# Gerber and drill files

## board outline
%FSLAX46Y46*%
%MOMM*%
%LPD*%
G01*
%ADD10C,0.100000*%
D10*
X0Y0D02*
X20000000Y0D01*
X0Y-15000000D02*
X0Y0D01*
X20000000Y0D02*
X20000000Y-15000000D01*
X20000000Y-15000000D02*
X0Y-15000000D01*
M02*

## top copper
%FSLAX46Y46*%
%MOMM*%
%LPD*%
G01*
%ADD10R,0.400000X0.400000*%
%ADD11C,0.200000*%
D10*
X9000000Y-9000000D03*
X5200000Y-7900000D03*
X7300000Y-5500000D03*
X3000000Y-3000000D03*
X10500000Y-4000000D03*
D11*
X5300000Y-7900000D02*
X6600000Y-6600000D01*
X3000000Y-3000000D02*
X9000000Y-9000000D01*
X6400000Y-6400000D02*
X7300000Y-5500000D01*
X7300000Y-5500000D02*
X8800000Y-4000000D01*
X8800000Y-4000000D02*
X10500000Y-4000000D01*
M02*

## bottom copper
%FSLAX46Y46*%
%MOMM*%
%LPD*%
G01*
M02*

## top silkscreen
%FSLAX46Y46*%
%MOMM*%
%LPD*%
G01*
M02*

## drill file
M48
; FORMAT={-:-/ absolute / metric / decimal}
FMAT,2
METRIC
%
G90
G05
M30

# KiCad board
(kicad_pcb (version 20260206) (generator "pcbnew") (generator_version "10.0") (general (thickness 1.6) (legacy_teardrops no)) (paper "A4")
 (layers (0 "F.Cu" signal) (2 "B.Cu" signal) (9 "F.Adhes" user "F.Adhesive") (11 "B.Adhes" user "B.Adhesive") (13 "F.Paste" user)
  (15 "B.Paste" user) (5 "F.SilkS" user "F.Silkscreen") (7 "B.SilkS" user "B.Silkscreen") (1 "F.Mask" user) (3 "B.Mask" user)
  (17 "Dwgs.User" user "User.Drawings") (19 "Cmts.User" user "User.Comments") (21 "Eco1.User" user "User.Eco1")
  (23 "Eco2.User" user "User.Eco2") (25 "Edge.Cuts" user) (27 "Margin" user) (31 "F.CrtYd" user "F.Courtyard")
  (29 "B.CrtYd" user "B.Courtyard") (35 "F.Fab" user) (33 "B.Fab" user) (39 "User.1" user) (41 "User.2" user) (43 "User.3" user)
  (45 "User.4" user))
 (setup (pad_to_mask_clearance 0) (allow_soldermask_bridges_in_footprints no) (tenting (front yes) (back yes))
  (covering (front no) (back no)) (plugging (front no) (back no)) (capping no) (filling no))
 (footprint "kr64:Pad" (layer "F.Cu") (at 9 9)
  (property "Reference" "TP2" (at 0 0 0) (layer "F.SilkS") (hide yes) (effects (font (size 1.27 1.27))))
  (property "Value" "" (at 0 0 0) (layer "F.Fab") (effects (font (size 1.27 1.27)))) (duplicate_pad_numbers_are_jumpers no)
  (pad "1" smd rect (at 0 0) (size 0.4 0.4) (layers "F.Cu" "F.Mask" "F.Paste") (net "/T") (thermal_bridge_angle 45)))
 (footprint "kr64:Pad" (layer "F.Cu") (at 5.2 7.9)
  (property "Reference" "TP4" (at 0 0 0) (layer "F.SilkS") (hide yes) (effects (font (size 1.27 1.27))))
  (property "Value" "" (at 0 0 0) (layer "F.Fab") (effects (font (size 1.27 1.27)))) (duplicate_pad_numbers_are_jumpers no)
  (pad "1" smd rect (at 0 0) (size 0.4 0.4) (layers "F.Cu" "F.Mask" "F.Paste") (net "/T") (thermal_bridge_angle 45)))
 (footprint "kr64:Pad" (layer "F.Cu") (at 7.3 5.5)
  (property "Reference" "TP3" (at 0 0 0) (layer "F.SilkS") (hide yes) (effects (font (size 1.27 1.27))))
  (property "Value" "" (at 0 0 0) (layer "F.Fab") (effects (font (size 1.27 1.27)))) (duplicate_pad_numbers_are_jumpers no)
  (pad "1" smd rect (at 0 0) (size 0.4 0.4) (layers "F.Cu" "F.Mask" "F.Paste") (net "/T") (thermal_bridge_angle 45)))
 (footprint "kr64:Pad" (layer "F.Cu") (at 3 3)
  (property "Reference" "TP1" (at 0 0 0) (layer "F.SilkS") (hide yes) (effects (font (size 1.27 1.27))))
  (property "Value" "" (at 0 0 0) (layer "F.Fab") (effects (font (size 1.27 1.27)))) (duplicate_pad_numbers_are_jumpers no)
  (pad "1" smd rect (at 0 0) (size 0.4 0.4) (layers "F.Cu" "F.Mask" "F.Paste") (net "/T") (thermal_bridge_angle 45)))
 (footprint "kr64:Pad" (layer "F.Cu") (at 10.5 4)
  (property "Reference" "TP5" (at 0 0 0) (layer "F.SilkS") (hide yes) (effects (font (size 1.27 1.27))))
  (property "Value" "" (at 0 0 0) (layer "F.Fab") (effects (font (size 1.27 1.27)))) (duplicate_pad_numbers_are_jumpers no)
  (pad "1" smd rect (at 0 0) (size 0.4 0.4) (layers "F.Cu" "F.Mask" "F.Paste") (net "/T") (thermal_bridge_angle 45)))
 (gr_line (start 0 0) (end 20 0) (stroke (width 0.1) (type default)) (layer "Edge.Cuts"))
 (gr_line (start 0 15) (end 0 0) (stroke (width 0.1) (type default)) (layer "Edge.Cuts"))
 (gr_line (start 20 0) (end 20 15) (stroke (width 0.1) (type default)) (layer "Edge.Cuts"))
 (gr_line (start 20 15) (end 0 15) (stroke (width 0.1) (type default)) (layer "Edge.Cuts"))
 (segment (start 5.3 7.9) (end 6.6 6.6) (width 0.2) (layer "F.Cu") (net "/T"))
 (segment (start 3 3) (end 9 9) (width 0.2) (layer "F.Cu") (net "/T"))
 (segment (start 6.4 6.4) (end 7.3 5.5) (width 0.2) (layer "F.Cu") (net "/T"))
 (segment (start 7.3 5.5) (end 8.8 4) (width 0.2) (layer "F.Cu") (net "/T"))
 (segment (start 8.8 4) (end 10.5 4) (width 0.2) (layer "F.Cu") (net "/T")))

